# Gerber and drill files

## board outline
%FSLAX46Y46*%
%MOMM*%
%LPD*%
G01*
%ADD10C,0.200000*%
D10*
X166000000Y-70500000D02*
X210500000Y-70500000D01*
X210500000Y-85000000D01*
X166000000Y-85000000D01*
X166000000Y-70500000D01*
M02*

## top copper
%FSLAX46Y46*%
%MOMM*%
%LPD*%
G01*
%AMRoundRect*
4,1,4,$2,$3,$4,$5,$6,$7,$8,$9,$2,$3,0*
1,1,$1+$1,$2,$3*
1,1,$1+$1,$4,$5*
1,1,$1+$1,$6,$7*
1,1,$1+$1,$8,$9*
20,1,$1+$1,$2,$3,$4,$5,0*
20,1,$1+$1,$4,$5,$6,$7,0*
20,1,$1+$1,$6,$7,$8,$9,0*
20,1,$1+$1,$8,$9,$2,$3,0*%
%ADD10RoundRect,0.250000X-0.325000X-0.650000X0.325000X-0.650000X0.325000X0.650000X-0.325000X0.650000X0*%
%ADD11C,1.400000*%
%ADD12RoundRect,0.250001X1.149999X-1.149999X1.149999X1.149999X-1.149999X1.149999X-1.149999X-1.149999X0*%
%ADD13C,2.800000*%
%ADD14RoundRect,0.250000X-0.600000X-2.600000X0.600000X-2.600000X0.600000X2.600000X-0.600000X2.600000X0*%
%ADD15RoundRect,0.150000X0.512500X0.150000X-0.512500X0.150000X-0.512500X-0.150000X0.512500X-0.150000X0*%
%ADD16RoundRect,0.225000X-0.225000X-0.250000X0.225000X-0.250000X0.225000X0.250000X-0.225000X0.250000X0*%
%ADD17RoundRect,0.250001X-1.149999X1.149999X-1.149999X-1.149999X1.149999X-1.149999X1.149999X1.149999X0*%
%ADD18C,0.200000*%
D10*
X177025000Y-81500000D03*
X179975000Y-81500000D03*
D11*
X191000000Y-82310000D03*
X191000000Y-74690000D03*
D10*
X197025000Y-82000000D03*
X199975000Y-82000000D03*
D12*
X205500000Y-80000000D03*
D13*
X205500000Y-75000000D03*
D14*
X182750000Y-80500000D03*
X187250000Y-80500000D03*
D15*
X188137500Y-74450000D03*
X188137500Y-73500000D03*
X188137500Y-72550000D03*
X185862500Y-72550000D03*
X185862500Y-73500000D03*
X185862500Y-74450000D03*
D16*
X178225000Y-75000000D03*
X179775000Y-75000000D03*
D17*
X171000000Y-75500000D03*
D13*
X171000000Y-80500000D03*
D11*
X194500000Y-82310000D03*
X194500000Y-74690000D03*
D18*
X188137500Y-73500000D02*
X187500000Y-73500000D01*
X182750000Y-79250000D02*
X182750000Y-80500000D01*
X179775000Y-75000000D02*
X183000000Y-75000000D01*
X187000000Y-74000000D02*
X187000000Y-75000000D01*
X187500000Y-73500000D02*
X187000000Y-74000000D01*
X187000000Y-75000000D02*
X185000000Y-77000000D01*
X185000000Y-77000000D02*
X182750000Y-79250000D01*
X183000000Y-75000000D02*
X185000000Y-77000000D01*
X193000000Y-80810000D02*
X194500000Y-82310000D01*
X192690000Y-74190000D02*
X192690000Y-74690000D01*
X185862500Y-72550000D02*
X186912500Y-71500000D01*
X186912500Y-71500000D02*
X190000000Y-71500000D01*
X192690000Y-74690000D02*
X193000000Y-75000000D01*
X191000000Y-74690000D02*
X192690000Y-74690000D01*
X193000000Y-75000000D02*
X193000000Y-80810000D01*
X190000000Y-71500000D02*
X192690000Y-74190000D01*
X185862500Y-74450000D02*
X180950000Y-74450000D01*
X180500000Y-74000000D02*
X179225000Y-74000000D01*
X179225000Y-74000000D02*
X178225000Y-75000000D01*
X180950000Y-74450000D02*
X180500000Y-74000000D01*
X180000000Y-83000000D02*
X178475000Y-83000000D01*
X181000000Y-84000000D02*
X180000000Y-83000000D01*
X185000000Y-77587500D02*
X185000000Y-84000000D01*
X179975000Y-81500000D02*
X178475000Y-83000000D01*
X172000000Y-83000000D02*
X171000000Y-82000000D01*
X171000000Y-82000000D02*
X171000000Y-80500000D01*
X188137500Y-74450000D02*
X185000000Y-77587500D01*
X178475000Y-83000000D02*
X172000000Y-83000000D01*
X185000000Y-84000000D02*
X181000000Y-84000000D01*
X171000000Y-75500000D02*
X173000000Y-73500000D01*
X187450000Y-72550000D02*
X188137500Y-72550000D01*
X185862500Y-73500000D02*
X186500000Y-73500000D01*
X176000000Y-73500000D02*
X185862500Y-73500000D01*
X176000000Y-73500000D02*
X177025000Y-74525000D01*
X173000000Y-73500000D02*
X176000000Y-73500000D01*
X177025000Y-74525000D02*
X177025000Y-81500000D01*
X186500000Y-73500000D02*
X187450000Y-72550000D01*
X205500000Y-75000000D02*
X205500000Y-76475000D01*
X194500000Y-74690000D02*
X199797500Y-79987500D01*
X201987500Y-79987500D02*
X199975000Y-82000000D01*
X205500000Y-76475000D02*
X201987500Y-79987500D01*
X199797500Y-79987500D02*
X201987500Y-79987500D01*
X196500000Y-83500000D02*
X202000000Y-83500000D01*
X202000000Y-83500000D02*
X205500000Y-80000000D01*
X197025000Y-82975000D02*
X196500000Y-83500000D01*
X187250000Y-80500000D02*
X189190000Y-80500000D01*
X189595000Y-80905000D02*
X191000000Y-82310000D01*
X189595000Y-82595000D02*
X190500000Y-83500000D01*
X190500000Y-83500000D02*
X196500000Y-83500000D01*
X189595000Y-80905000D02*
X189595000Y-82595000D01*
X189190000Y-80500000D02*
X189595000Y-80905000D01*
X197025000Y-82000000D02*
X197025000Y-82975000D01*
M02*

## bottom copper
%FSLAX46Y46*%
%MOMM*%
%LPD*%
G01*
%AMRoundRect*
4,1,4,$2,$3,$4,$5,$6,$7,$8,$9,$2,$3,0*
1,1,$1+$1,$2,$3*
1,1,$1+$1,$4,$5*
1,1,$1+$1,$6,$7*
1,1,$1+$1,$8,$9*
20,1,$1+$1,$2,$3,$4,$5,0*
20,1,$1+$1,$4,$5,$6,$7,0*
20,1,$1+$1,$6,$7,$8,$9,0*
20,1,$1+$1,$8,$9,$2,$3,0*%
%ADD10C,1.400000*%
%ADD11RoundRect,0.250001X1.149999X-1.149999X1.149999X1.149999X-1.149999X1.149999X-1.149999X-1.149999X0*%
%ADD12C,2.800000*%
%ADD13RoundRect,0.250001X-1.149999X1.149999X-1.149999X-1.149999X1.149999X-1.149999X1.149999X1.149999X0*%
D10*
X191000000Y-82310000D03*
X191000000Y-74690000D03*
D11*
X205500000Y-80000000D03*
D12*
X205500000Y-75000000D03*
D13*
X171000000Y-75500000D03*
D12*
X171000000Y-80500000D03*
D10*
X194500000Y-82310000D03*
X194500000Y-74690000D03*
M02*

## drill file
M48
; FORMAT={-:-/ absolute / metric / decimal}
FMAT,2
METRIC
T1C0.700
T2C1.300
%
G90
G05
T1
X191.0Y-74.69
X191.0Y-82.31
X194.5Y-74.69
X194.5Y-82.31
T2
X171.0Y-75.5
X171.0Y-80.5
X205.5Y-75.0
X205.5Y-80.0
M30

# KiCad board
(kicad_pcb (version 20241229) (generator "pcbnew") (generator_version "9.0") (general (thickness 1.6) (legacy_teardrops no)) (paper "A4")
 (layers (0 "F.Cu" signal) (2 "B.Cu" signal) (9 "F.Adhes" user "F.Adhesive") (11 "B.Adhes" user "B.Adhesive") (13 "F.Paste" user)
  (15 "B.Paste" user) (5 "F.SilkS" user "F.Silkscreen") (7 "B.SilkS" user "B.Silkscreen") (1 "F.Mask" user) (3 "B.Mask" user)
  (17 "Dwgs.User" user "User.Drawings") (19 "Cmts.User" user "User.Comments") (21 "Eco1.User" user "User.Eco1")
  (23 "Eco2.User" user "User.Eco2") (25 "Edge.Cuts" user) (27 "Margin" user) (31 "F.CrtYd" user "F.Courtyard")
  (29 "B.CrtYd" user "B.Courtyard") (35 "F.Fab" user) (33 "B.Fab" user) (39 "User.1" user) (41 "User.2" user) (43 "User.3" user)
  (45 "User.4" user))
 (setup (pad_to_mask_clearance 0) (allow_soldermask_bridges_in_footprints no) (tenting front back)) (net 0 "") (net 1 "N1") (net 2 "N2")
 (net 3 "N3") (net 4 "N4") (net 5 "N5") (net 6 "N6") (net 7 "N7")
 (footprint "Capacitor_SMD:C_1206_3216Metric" (layer "F.Cu") (at 178.5 81.5)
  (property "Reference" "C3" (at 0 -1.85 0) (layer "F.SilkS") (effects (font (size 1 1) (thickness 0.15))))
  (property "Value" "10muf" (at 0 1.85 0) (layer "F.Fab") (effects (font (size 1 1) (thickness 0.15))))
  (pad "1" smd roundrect (at -1.475 0) (size 1.15 1.8) (layers "F.Cu" "F.Mask" "F.Paste") (roundrect_rratio 0.217391) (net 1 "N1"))
  (pad "2" smd roundrect (at 1.475 0) (size 1.15 1.8) (layers "F.Cu" "F.Mask" "F.Paste") (roundrect_rratio 0.217391) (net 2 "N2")))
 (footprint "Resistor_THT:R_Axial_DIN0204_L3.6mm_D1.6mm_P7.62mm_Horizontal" (layer "F.Cu") (at 191 82.31 90)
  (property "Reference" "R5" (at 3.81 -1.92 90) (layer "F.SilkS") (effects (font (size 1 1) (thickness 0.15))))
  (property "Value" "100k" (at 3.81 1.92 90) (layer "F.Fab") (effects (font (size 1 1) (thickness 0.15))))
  (pad "1" thru_hole circle (at 0 0 90) (size 1.4 1.4) (drill 0.7) (layers "*.Cu" "*.Mask") (remove_unused_layers no) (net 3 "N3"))
  (pad "2" thru_hole circle (at 7.62 0 90) (size 1.4 1.4) (drill 0.7) (layers "*.Cu" "*.Mask") (remove_unused_layers no) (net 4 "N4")))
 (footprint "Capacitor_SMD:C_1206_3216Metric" (layer "F.Cu") (at 198.5 82)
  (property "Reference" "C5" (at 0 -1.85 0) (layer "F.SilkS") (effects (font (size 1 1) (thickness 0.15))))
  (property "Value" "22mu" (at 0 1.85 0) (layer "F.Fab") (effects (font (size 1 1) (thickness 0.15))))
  (pad "1" smd roundrect (at -1.475 0) (size 1.15 1.8) (layers "F.Cu" "F.Mask" "F.Paste") (roundrect_rratio 0.217391) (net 4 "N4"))
  (pad "2" smd roundrect (at 1.475 0) (size 1.15 1.8) (layers "F.Cu" "F.Mask" "F.Paste") (roundrect_rratio 0.217391) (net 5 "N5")))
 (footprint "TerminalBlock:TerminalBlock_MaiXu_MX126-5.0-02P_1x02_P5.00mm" (layer "F.Cu") (at 205.5 80 90)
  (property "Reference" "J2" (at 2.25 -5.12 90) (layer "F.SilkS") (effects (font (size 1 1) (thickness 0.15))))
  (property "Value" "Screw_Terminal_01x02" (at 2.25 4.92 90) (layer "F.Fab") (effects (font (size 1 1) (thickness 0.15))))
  (pad "1" thru_hole roundrect (at 0 0 90) (size 2.8 2.8) (drill 1.3) (layers "*.Cu" "*.Mask") (remove_unused_layers no)
   (roundrect_rratio 0.089286) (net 4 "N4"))
  (pad "2" thru_hole circle (at 5 0 90) (size 2.8 2.8) (drill 1.3) (layers "*.Cu" "*.Mask") (remove_unused_layers no) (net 5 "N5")))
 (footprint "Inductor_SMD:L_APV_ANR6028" (layer "F.Cu") (at 185 80.5)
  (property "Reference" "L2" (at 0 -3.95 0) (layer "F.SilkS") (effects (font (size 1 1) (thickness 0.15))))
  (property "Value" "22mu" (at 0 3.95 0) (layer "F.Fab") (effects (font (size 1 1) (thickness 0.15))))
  (pad "1" smd roundrect (at -2.25 0) (size 1.7 5.7) (layers "F.Cu" "F.Mask" "F.Paste") (roundrect_rratio 0.147059) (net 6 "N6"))
  (pad "2" smd roundrect (at 2.25 0) (size 1.7 5.7) (layers "F.Cu" "F.Mask" "F.Paste") (roundrect_rratio 0.147059) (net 4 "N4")))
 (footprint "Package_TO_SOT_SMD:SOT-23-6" (layer "F.Cu") (at 187 73.5 180)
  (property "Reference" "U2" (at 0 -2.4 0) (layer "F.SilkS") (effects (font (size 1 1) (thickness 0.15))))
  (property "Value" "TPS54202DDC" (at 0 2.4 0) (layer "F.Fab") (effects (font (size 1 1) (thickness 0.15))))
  (pad "1" smd roundrect (at -1.1375 -0.95 180) (size 1.325 0.6) (layers "F.Cu" "F.Mask" "F.Paste") (roundrect_rratio 0.25) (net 2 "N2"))
  (pad "2" smd roundrect (at -1.1375 0 180) (size 1.325 0.6) (layers "F.Cu" "F.Mask" "F.Paste") (roundrect_rratio 0.25) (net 6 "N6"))
  (pad "3" smd roundrect (at -1.1375 0.95 180) (size 1.325 0.6) (layers "F.Cu" "F.Mask" "F.Paste") (roundrect_rratio 0.25) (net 1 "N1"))
  (pad "4" smd roundrect (at 1.1375 0.95 180) (size 1.325 0.6) (layers "F.Cu" "F.Mask" "F.Paste") (roundrect_rratio 0.25) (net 3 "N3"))
  (pad "5" smd roundrect (at 1.1375 0 180) (size 1.325 0.6) (layers "F.Cu" "F.Mask" "F.Paste") (roundrect_rratio 0.25) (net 1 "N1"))
  (pad "6" smd roundrect (at 1.1375 -0.95 180) (size 1.325 0.6) (layers "F.Cu" "F.Mask" "F.Paste") (roundrect_rratio 0.25) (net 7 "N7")))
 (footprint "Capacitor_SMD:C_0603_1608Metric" (layer "F.Cu") (at 179 75)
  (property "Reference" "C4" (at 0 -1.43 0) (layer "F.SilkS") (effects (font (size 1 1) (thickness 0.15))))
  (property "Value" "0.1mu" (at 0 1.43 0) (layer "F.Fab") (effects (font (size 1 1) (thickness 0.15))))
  (pad "1" smd roundrect (at -0.775 0) (size 0.9 0.95) (layers "F.Cu" "F.Mask" "F.Paste") (roundrect_rratio 0.25) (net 7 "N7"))
  (pad "2" smd roundrect (at 0.775 0) (size 0.9 0.95) (layers "F.Cu" "F.Mask" "F.Paste") (roundrect_rratio 0.25) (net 6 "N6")))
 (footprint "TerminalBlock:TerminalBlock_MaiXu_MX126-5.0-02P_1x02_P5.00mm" (layer "F.Cu") (at 171 75.5 -90)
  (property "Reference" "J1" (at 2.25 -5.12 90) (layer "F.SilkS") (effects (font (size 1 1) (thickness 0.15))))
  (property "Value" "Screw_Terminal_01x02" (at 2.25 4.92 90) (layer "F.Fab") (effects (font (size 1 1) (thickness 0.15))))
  (pad "1" thru_hole roundrect (at 0 0 270) (size 2.8 2.8) (drill 1.3) (layers "*.Cu" "*.Mask") (remove_unused_layers no)
   (roundrect_rratio 0.089286) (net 1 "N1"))
  (pad "2" thru_hole circle (at 5 0 270) (size 2.8 2.8) (drill 1.3) (layers "*.Cu" "*.Mask") (remove_unused_layers no) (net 2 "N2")))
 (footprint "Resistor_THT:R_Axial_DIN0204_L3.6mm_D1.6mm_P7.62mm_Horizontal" (layer "F.Cu") (at 194.5 82.31 90)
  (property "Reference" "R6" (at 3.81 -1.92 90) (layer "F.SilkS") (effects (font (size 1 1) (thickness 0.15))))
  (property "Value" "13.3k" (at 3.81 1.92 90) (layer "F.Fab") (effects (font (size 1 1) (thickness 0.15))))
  (pad "1" thru_hole circle (at 0 0 90) (size 1.4 1.4) (drill 0.7) (layers "*.Cu" "*.Mask") (remove_unused_layers no) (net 3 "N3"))
  (pad "2" thru_hole circle (at 7.62 0 90) (size 1.4 1.4) (drill 0.7) (layers "*.Cu" "*.Mask") (remove_unused_layers no) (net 5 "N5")))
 (gr_rect (start 166 70.5) (end 210.5 85) (stroke (width 0.2) (type solid)) (fill no) (layer "Edge.Cuts"))
 (segment (start 188.1375 73.5) (end 187.5 73.5) (width 0.2) (layer "F.Cu") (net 6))
 (segment (start 182.75 79.25) (end 182.75 80.5) (width 0.2) (layer "F.Cu") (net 6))
 (segment (start 179.775 75) (end 183 75) (width 0.2) (layer "F.Cu") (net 6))
 (segment (start 187 74) (end 187 75) (width 0.2) (layer "F.Cu") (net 6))
 (segment (start 187.5 73.5) (end 187 74) (width 0.2) (layer "F.Cu") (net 6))
 (segment (start 187 75) (end 185 77) (width 0.2) (layer "F.Cu") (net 6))
 (segment (start 185 77) (end 182.75 79.25) (width 0.2) (layer "F.Cu") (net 6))
 (segment (start 183 75) (end 185 77) (width 0.2) (layer "F.Cu") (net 6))
 (segment (start 193 80.81) (end 194.5 82.31) (width 0.2) (layer "F.Cu") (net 3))
 (segment (start 192.69 74.19) (end 192.69 74.69) (width 0.2) (layer "F.Cu") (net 3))
 (segment (start 185.8625 72.55) (end 186.9125 71.5) (width 0.2) (layer "F.Cu") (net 3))
 (segment (start 186.9125 71.5) (end 190 71.5) (width 0.2) (layer "F.Cu") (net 3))
 (segment (start 192.69 74.69) (end 193 75) (width 0.2) (layer "F.Cu") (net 3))
 (segment (start 191 74.69) (end 192.69 74.69) (width 0.2) (layer "F.Cu") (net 3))
 (segment (start 193 75) (end 193 80.81) (width 0.2) (layer "F.Cu") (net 3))
 (segment (start 190 71.5) (end 192.69 74.19) (width 0.2) (layer "F.Cu") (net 3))
 (segment (start 185.8625 74.45) (end 180.95 74.45) (width 0.2) (layer "F.Cu") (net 7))
 (segment (start 180.5 74) (end 179.225 74) (width 0.2) (layer "F.Cu") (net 7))
 (segment (start 179.225 74) (end 178.225 75) (width 0.2) (layer "F.Cu") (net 7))
 (segment (start 180.95 74.45) (end 180.5 74) (width 0.2) (layer "F.Cu") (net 7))
 (segment (start 180 83) (end 178.475 83) (width 0.2) (layer "F.Cu") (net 2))
 (segment (start 181 84) (end 180 83) (width 0.2) (layer "F.Cu") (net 2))
 (segment (start 185 77.5875) (end 185 84) (width 0.2) (layer "F.Cu") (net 2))
 (segment (start 179.975 81.5) (end 178.475 83) (width 0.2) (layer "F.Cu") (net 2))
 (segment (start 172 83) (end 171 82) (width 0.2) (layer "F.Cu") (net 2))
 (segment (start 171 82) (end 171 80.5) (width 0.2) (layer "F.Cu") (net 2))
 (segment (start 188.1375 74.45) (end 185 77.5875) (width 0.2) (layer "F.Cu") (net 2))
 (segment (start 178.475 83) (end 172 83) (width 0.2) (layer "F.Cu") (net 2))
 (segment (start 185 84) (end 181 84) (width 0.2) (layer "F.Cu") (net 2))
 (segment (start 171 75.5) (end 173 73.5) (width 0.2) (layer "F.Cu") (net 1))
 (segment (start 187.45 72.55) (end 188.1375 72.55) (width 0.2) (layer "F.Cu") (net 1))
 (segment (start 185.8625 73.5) (end 186.5 73.5) (width 0.2) (layer "F.Cu") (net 1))
 (segment (start 176 73.5) (end 185.8625 73.5) (width 0.2) (layer "F.Cu") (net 1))
 (segment (start 176 73.5) (end 177.025 74.525) (width 0.2) (layer "F.Cu") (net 1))
 (segment (start 173 73.5) (end 176 73.5) (width 0.2) (layer "F.Cu") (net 1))
 (segment (start 177.025 74.525) (end 177.025 81.5) (width 0.2) (layer "F.Cu") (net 1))
 (segment (start 186.5 73.5) (end 187.45 72.55) (width 0.2) (layer "F.Cu") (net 1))
 (segment (start 205.5 75) (end 205.5 76.475) (width 0.2) (layer "F.Cu") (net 5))
 (segment (start 194.5 74.69) (end 199.7975 79.9875) (width 0.2) (layer "F.Cu") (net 5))
 (segment (start 201.9875 79.9875) (end 199.975 82) (width 0.2) (layer "F.Cu") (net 5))
 (segment (start 205.5 76.475) (end 201.9875 79.9875) (width 0.2) (layer "F.Cu") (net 5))
 (segment (start 199.7975 79.9875) (end 201.9875 79.9875) (width 0.2) (layer "F.Cu") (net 5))
 (segment (start 196.5 83.5) (end 202 83.5) (width 0.2) (layer "F.Cu") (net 4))
 (segment (start 202 83.5) (end 205.5 80) (width 0.2) (layer "F.Cu") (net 4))
 (segment (start 197.025 82.975) (end 196.5 83.5) (width 0.2) (layer "F.Cu") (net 4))
 (segment (start 187.25 80.5) (end 189.19 80.5) (width 0.2) (layer "F.Cu") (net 4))
 (segment (start 189.595 80.905) (end 191 82.31) (width 0.2) (layer "F.Cu") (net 4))
 (segment (start 189.595 82.595) (end 190.5 83.5) (width 0.2) (layer "F.Cu") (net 4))
 (segment (start 190.5 83.5) (end 196.5 83.5) (width 0.2) (layer "F.Cu") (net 4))
 (segment (start 189.595 80.905) (end 189.595 82.595) (width 0.2) (layer "F.Cu") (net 4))
 (segment (start 189.19 80.5) (end 189.595 80.905) (width 0.2) (layer "F.Cu") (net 4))
 (segment (start 197.025 82) (end 197.025 82.975) (width 0.2) (layer "F.Cu") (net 4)))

